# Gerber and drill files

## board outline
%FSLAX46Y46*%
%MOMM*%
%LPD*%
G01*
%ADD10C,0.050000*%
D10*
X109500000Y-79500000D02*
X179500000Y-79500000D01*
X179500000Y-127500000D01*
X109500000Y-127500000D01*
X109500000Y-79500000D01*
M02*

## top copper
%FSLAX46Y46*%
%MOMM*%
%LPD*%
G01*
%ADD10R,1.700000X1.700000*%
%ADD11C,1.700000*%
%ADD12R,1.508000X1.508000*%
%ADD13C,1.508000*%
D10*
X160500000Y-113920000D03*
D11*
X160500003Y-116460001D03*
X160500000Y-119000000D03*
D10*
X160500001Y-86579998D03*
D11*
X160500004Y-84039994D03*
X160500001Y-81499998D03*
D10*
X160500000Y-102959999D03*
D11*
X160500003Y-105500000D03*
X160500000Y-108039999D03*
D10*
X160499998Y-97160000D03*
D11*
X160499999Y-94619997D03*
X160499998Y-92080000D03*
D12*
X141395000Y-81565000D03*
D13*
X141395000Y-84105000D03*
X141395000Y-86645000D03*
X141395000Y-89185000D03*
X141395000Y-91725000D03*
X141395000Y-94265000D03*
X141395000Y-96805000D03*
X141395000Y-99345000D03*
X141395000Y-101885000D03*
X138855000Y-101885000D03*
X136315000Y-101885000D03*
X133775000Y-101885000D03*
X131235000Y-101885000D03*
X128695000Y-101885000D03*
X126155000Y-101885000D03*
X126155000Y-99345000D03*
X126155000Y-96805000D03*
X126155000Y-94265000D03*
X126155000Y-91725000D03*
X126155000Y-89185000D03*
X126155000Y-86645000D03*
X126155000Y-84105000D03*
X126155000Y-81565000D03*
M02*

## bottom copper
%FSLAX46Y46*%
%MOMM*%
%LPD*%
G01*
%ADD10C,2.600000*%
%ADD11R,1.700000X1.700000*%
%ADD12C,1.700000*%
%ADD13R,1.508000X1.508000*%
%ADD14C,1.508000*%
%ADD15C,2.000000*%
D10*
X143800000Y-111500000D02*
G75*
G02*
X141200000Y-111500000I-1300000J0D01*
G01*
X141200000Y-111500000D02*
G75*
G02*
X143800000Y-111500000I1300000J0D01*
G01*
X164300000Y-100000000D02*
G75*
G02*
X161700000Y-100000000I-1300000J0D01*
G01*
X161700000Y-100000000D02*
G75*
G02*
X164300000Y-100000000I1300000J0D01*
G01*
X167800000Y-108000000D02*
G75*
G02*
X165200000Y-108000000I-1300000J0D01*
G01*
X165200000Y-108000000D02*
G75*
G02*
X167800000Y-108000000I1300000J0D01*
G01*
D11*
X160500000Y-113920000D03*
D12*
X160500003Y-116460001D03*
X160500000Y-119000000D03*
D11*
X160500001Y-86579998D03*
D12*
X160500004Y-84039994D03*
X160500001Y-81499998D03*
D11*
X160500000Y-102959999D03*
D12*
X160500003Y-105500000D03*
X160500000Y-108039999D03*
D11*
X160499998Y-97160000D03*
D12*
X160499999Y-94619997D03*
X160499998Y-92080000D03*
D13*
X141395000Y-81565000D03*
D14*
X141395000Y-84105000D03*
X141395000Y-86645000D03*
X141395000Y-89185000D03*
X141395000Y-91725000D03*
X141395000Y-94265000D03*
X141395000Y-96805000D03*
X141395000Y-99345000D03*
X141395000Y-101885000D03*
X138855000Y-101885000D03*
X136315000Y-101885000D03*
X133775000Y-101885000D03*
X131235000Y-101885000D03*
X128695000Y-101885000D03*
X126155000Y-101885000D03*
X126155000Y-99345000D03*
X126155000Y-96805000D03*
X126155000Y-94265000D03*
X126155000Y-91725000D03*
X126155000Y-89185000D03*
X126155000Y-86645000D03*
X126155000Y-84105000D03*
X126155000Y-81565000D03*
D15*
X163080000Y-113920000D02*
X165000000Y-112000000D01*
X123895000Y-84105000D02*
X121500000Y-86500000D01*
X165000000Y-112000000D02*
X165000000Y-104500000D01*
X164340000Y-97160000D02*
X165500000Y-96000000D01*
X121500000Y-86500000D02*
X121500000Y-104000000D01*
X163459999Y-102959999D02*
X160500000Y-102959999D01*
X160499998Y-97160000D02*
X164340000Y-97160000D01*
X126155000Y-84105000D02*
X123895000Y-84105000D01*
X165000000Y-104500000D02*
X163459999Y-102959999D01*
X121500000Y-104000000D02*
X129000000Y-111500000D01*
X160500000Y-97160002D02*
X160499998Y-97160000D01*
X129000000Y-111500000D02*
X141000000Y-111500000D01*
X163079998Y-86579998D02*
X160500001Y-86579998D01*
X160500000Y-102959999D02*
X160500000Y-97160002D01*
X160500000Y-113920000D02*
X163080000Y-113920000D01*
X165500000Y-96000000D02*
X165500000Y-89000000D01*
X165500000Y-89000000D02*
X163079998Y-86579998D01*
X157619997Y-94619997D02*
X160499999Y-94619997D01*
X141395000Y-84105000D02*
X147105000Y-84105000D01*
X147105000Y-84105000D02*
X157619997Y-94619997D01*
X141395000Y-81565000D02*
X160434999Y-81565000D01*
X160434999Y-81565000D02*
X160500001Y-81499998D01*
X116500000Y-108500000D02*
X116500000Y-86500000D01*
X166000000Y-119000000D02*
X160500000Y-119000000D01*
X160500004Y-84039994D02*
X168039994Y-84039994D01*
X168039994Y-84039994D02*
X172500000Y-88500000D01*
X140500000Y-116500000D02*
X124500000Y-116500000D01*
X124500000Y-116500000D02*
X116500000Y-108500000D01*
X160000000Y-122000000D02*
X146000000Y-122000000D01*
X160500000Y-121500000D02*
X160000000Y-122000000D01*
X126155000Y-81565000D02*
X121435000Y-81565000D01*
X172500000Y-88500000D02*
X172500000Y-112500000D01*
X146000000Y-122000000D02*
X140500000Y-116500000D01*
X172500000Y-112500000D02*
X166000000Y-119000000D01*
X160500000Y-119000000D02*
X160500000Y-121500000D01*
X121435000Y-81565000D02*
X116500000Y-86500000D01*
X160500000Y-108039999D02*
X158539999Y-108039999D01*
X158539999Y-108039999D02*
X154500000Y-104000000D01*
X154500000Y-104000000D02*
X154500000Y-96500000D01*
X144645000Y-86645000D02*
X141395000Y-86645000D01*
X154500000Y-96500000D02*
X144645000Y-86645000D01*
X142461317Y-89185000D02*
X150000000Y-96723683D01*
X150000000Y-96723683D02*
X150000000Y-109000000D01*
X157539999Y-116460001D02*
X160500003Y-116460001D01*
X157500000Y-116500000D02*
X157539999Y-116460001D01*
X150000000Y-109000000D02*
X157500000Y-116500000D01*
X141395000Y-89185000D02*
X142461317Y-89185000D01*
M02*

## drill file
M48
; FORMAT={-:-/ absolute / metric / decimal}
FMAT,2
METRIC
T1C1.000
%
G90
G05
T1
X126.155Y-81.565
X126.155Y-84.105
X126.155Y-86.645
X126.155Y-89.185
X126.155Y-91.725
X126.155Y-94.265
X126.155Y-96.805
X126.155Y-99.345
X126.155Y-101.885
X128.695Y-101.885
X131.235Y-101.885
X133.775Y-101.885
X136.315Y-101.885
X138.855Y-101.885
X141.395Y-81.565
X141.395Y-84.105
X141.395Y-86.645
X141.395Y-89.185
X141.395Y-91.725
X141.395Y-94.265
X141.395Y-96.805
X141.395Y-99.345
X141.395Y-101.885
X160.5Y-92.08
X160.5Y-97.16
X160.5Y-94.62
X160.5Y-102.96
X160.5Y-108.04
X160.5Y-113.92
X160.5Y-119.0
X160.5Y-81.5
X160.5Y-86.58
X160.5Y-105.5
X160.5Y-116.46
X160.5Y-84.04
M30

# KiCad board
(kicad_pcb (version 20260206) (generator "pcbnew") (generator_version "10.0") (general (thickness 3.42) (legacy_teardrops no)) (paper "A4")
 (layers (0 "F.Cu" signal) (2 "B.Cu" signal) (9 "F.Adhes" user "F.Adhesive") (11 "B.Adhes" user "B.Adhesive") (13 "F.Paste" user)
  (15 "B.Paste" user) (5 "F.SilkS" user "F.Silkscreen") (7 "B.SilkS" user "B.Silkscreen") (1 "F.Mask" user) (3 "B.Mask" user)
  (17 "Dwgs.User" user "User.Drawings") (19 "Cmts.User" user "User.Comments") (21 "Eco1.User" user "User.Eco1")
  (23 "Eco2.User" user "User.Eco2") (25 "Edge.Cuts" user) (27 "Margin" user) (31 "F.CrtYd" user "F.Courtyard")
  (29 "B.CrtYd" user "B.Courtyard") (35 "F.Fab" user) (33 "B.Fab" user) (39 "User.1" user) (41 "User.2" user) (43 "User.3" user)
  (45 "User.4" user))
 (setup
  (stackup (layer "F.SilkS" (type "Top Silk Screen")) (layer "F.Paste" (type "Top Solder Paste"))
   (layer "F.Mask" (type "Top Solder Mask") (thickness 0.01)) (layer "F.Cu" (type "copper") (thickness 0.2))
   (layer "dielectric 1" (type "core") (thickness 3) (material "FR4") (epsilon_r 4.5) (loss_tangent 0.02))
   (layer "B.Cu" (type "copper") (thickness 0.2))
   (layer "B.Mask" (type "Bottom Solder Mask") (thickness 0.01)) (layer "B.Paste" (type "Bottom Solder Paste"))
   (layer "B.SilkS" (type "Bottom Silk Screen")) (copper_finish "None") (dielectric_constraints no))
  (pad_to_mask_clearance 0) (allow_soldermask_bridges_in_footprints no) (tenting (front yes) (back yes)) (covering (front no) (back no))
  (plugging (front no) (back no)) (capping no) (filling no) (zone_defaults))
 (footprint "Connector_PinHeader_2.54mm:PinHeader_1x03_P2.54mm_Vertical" (layer "F.Cu") (at 160.5 113.92)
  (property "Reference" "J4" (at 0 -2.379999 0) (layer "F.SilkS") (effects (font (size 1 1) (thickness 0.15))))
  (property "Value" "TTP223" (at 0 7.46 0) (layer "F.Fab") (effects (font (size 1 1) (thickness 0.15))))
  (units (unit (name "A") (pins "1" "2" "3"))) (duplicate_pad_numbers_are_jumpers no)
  (pad "1" thru_hole rect (at 0 0) (size 1.7 1.7) (drill 1) (layers "*.Cu" "*.Mask") (remove_unused_layers no) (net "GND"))
  (pad "2" thru_hole circle (at 0.000003 2.540001) (size 1.7 1.7) (drill 1) (layers "*.Cu" "*.Mask") (remove_unused_layers no) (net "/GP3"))
  (pad "3" thru_hole circle (at 0 5.08) (size 1.7 1.7) (drill 1) (layers "*.Cu" "*.Mask") (remove_unused_layers no) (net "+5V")))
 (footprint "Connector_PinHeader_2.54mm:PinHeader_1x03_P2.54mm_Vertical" (layer "F.Cu") (at 160.500001 86.579998 180)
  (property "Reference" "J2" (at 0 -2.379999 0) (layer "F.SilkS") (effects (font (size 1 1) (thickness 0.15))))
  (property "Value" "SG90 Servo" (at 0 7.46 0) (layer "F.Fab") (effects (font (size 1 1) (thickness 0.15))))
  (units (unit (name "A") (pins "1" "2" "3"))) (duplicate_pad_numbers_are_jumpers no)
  (pad "1" thru_hole rect (at 0 0 180) (size 1.7 1.7) (drill 1) (layers "*.Cu" "*.Mask") (remove_unused_layers no) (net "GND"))
  (pad "2" thru_hole circle (at -0.000003 2.540004 180) (size 1.7 1.7) (drill 1) (layers "*.Cu" "*.Mask") (remove_unused_layers no)
   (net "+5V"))
  (pad "3" thru_hole circle (at 0 5.08 180) (size 1.7 1.7) (drill 1) (layers "*.Cu" "*.Mask") (remove_unused_layers no) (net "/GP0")))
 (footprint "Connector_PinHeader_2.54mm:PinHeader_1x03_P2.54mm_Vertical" (layer "F.Cu") (at 160.5 102.959999)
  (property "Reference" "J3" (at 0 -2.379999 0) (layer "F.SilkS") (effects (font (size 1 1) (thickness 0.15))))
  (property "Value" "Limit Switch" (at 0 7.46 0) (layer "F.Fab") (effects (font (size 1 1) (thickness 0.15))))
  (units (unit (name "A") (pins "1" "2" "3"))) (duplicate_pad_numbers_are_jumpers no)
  (pad "1" thru_hole rect (at 0 0) (size 1.7 1.7) (drill 1) (layers "*.Cu" "*.Mask") (remove_unused_layers no) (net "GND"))
  (pad "2" thru_hole circle (at 0.000003 2.540001) (size 1.7 1.7) (drill 1) (layers "*.Cu" "*.Mask") (remove_unused_layers no)
   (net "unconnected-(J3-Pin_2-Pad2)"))
  (pad "3" thru_hole circle (at 0 5.08) (size 1.7 1.7) (drill 1) (layers "*.Cu" "*.Mask") (remove_unused_layers no) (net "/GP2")))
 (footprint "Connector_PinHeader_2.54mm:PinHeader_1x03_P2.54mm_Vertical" (layer "F.Cu") (at 160.499998 97.16 180)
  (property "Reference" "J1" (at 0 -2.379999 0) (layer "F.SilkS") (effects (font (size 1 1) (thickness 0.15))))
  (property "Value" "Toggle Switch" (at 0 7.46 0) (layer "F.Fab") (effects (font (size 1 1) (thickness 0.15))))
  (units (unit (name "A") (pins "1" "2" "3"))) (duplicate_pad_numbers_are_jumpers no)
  (pad "1" thru_hole rect (at 0 0 180) (size 1.7 1.7) (drill 1) (layers "*.Cu" "*.Mask") (remove_unused_layers no) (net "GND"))
  (pad "2" thru_hole circle (at -0.000001 2.540003 180) (size 1.7 1.7) (drill 1) (layers "*.Cu" "*.Mask") (remove_unused_layers no)
   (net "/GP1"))
  (pad "3" thru_hole circle (at 0 5.08 180) (size 1.7 1.7) (drill 1) (layers "*.Cu" "*.Mask") (remove_unused_layers no)
   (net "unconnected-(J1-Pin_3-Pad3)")))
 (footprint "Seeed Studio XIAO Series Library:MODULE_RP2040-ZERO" (layer "F.Cu") (at 133.775 91.725)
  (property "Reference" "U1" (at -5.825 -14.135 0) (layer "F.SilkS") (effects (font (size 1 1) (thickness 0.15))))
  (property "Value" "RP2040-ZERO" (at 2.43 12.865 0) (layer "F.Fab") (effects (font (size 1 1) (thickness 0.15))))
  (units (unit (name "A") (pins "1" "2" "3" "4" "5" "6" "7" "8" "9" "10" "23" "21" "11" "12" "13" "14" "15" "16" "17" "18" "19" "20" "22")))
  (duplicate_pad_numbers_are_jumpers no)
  (pad "1" thru_hole rect (at 7.62 -10.16) (size 1.508 1.508) (drill 1) (layers "*.Cu" "*.Mask") (remove_unused_layers no) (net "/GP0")
   (solder_mask_margin 0.102))
  (pad "2" thru_hole circle (at 7.62 -7.62) (size 1.508 1.508) (drill 1) (layers "*.Cu" "*.Mask") (remove_unused_layers no) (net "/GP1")
   (solder_mask_margin 0.102))
  (pad "3" thru_hole circle (at 7.62 -5.08) (size 1.508 1.508) (drill 1) (layers "*.Cu" "*.Mask") (remove_unused_layers no) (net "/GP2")
   (solder_mask_margin 0.102))
  (pad "4" thru_hole circle (at 7.62 -2.54) (size 1.508 1.508) (drill 1) (layers "*.Cu" "*.Mask") (remove_unused_layers no) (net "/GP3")
   (solder_mask_margin 0.102))
  (pad "5" thru_hole circle (at 7.62 0) (size 1.508 1.508) (drill 1) (layers "*.Cu" "*.Mask") (remove_unused_layers no)
   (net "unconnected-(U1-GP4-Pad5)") (solder_mask_margin 0.102))
  (pad "6" thru_hole circle (at 7.62 2.54) (size 1.508 1.508) (drill 1) (layers "*.Cu" "*.Mask") (remove_unused_layers no)
   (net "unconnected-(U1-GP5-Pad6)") (solder_mask_margin 0.102))
  (pad "7" thru_hole circle (at 7.62 5.08) (size 1.508 1.508) (drill 1) (layers "*.Cu" "*.Mask") (remove_unused_layers no)
   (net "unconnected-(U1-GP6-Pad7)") (solder_mask_margin 0.102))
  (pad "8" thru_hole circle (at 7.62 7.62) (size 1.508 1.508) (drill 1) (layers "*.Cu" "*.Mask") (remove_unused_layers no)
   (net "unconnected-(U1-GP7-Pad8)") (solder_mask_margin 0.102))
  (pad "9" thru_hole circle (at 7.62 10.16) (size 1.508 1.508) (drill 1) (layers "*.Cu" "*.Mask") (remove_unused_layers no)
   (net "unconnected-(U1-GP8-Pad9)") (solder_mask_margin 0.102))
  (pad "10" thru_hole circle (at 5.08 10.16) (size 1.508 1.508) (drill 1) (layers "*.Cu" "*.Mask") (remove_unused_layers no)
   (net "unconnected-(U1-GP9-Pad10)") (solder_mask_margin 0.102))
  (pad "11" thru_hole circle (at 2.54 10.16) (size 1.508 1.508) (drill 1) (layers "*.Cu" "*.Mask") (remove_unused_layers no)
   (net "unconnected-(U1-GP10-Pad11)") (solder_mask_margin 0.102))
  (pad "12" thru_hole circle (at 0 10.16) (size 1.508 1.508) (drill 1) (layers "*.Cu" "*.Mask") (remove_unused_layers no)
   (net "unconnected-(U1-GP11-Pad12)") (solder_mask_margin 0.102))
  (pad "13" thru_hole circle (at -2.54 10.16) (size 1.508 1.508) (drill 1) (layers "*.Cu" "*.Mask") (remove_unused_layers no)
   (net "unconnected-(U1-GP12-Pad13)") (solder_mask_margin 0.102))
  (pad "14" thru_hole circle (at -5.08 10.16) (size 1.508 1.508) (drill 1) (layers "*.Cu" "*.Mask") (remove_unused_layers no)
   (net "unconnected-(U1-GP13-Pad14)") (solder_mask_margin 0.102))
  (pad "15" thru_hole circle (at -7.62 10.16) (size 1.508 1.508) (drill 1) (layers "*.Cu" "*.Mask") (remove_unused_layers no)
   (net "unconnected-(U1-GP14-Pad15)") (solder_mask_margin 0.102))
  (pad "16" thru_hole circle (at -7.62 7.62) (size 1.508 1.508) (drill 1) (layers "*.Cu" "*.Mask") (remove_unused_layers no)
   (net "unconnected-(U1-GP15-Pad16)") (solder_mask_margin 0.102))
  (pad "17" thru_hole circle (at -7.62 5.08) (size 1.508 1.508) (drill 1) (layers "*.Cu" "*.Mask") (remove_unused_layers no)
   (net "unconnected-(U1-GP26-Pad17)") (solder_mask_margin 0.102))
  (pad "18" thru_hole circle (at -7.62 2.54) (size 1.508 1.508) (drill 1) (layers "*.Cu" "*.Mask") (remove_unused_layers no)
   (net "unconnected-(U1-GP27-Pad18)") (solder_mask_margin 0.102))
  (pad "19" thru_hole circle (at -7.62 0) (size 1.508 1.508) (drill 1) (layers "*.Cu" "*.Mask") (remove_unused_layers no)
   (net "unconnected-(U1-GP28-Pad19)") (solder_mask_margin 0.102))
  (pad "20" thru_hole circle (at -7.62 -2.54) (size 1.508 1.508) (drill 1) (layers "*.Cu" "*.Mask") (remove_unused_layers no)
   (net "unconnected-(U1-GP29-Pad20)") (solder_mask_margin 0.102))
  (pad "21" thru_hole circle (at -7.62 -5.08) (size 1.508 1.508) (drill 1) (layers "*.Cu" "*.Mask") (remove_unused_layers no)
   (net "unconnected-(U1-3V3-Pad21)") (solder_mask_margin 0.102))
  (pad "22" thru_hole circle (at -7.62 -7.62) (size 1.508 1.508) (drill 1) (layers "*.Cu" "*.Mask") (remove_unused_layers no) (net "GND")
   (solder_mask_margin 0.102))
  (pad "23" thru_hole circle (at -7.62 -10.16) (size 1.508 1.508) (drill 1) (layers "*.Cu" "*.Mask") (remove_unused_layers no) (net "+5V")
   (solder_mask_margin 0.102)))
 (gr_circle (center 142.5 111.5) (end 145 111.5) (stroke (width 0.2) (type solid)) (fill yes) (layer "B.Cu") (net "GND"))
 (gr_circle (center 163 100) (end 165.5 100) (stroke (width 0.2) (type solid)) (fill yes) (layer "B.Cu") (net "GND"))
 (gr_circle (center 166.5 108) (end 169 108) (stroke (width 0.2) (type solid)) (fill yes) (layer "B.Cu") (net "GND"))
 (gr_rect (start 109.5 79.5) (end 179.5 127.5) (stroke (width 0.05) (type default)) (fill no) (layer "Edge.Cuts"))
 (segment (start 163.08 113.92) (end 165 112) (width 2) (layer "B.Cu") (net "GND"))
 (segment (start 123.895 84.105) (end 121.5 86.5) (width 2) (layer "B.Cu") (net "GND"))
 (segment (start 165 112) (end 165 104.5) (width 2) (layer "B.Cu") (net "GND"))
 (segment (start 164.34 97.16) (end 165.5 96) (width 2) (layer "B.Cu") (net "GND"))
 (segment (start 121.5 86.5) (end 121.5 104) (width 2) (layer "B.Cu") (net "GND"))
 (segment (start 163.459999 102.959999) (end 160.5 102.959999) (width 2) (layer "B.Cu") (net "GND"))
 (segment (start 160.499998 97.16) (end 164.34 97.16) (width 2) (layer "B.Cu") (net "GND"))
 (segment (start 126.155 84.105) (end 123.895 84.105) (width 2) (layer "B.Cu") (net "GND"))
 (segment (start 165 104.5) (end 163.459999 102.959999) (width 2) (layer "B.Cu") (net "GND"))
 (segment (start 121.5 104) (end 129 111.5) (width 2) (layer "B.Cu") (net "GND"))
 (segment (start 160.5 97.160002) (end 160.499998 97.16) (width 2) (layer "B.Cu") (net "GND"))
 (segment (start 129 111.5) (end 141 111.5) (width 2) (layer "B.Cu") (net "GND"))
 (segment (start 163.079998 86.579998) (end 160.500001 86.579998) (width 2) (layer "B.Cu") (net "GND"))
 (segment (start 160.5 102.959999) (end 160.5 97.160002) (width 2) (layer "B.Cu") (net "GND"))
 (segment (start 160.5 113.92) (end 163.08 113.92) (width 2) (layer "B.Cu") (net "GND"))
 (segment (start 165.5 96) (end 165.5 89) (width 2) (layer "B.Cu") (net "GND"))
 (segment (start 165.5 89) (end 163.079998 86.579998) (width 2) (layer "B.Cu") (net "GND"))
 (segment (start 157.619997 94.619997) (end 160.499999 94.619997) (width 2) (layer "B.Cu") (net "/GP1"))
 (segment (start 141.395 84.105) (end 147.105 84.105) (width 2) (layer "B.Cu") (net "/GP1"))
 (segment (start 147.105 84.105) (end 157.619997 94.619997) (width 2) (layer "B.Cu") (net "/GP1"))
 (segment (start 141.395 81.565) (end 160.434999 81.565) (width 2) (layer "B.Cu") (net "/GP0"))
 (segment (start 160.434999 81.565) (end 160.500001 81.499998) (width 2) (layer "B.Cu") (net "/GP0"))
 (segment (start 116.5 108.5) (end 116.5 86.5) (width 2) (layer "B.Cu") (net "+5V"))
 (segment (start 166 119) (end 160.5 119) (width 2) (layer "B.Cu") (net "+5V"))
 (segment (start 160.500004 84.039994) (end 168.039994 84.039994) (width 2) (layer "B.Cu") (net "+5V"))
 (segment (start 168.039994 84.039994) (end 172.5 88.5) (width 2) (layer "B.Cu") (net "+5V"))
 (segment (start 140.5 116.5) (end 124.5 116.5) (width 2) (layer "B.Cu") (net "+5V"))
 (segment (start 124.5 116.5) (end 116.5 108.5) (width 2) (layer "B.Cu") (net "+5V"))
 (segment (start 160 122) (end 146 122) (width 2) (layer "B.Cu") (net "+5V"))
 (segment (start 160.5 121.5) (end 160 122) (width 2) (layer "B.Cu") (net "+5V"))
 (segment (start 126.155 81.565) (end 121.435 81.565) (width 2) (layer "B.Cu") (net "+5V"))
 (segment (start 172.5 88.5) (end 172.5 112.5) (width 2) (layer "B.Cu") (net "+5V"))
 (segment (start 146 122) (end 140.5 116.5) (width 2) (layer "B.Cu") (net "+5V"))
 (segment (start 172.5 112.5) (end 166 119) (width 2) (layer "B.Cu") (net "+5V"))
 (segment (start 160.5 119) (end 160.5 121.5) (width 2) (layer "B.Cu") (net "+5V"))
 (segment (start 121.435 81.565) (end 116.5 86.5) (width 2) (layer "B.Cu") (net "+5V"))
 (segment (start 160.5 108.039999) (end 158.539999 108.039999) (width 2) (layer "B.Cu") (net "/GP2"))
 (segment (start 158.539999 108.039999) (end 154.5 104) (width 2) (layer "B.Cu") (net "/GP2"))
 (segment (start 154.5 104) (end 154.5 96.5) (width 2) (layer "B.Cu") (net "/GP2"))
 (segment (start 144.645 86.645) (end 141.395 86.645) (width 2) (layer "B.Cu") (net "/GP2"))
 (segment (start 154.5 96.5) (end 144.645 86.645) (width 2) (layer "B.Cu") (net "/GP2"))
 (segment (start 142.461317 89.185) (end 150 96.723683) (width 2) (layer "B.Cu") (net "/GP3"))
 (segment (start 150 96.723683) (end 150 109) (width 2) (layer "B.Cu") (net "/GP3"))
 (segment (start 157.539999 116.460001) (end 160.500003 116.460001) (width 2) (layer "B.Cu") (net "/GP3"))
 (segment (start 157.5 116.5) (end 157.539999 116.460001) (width 2) (layer "B.Cu") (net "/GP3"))
 (segment (start 150 109) (end 157.5 116.5) (width 2) (layer "B.Cu") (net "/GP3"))
 (segment (start 141.395 89.185) (end 142.461317 89.185) (width 2) (layer "B.Cu") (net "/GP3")))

